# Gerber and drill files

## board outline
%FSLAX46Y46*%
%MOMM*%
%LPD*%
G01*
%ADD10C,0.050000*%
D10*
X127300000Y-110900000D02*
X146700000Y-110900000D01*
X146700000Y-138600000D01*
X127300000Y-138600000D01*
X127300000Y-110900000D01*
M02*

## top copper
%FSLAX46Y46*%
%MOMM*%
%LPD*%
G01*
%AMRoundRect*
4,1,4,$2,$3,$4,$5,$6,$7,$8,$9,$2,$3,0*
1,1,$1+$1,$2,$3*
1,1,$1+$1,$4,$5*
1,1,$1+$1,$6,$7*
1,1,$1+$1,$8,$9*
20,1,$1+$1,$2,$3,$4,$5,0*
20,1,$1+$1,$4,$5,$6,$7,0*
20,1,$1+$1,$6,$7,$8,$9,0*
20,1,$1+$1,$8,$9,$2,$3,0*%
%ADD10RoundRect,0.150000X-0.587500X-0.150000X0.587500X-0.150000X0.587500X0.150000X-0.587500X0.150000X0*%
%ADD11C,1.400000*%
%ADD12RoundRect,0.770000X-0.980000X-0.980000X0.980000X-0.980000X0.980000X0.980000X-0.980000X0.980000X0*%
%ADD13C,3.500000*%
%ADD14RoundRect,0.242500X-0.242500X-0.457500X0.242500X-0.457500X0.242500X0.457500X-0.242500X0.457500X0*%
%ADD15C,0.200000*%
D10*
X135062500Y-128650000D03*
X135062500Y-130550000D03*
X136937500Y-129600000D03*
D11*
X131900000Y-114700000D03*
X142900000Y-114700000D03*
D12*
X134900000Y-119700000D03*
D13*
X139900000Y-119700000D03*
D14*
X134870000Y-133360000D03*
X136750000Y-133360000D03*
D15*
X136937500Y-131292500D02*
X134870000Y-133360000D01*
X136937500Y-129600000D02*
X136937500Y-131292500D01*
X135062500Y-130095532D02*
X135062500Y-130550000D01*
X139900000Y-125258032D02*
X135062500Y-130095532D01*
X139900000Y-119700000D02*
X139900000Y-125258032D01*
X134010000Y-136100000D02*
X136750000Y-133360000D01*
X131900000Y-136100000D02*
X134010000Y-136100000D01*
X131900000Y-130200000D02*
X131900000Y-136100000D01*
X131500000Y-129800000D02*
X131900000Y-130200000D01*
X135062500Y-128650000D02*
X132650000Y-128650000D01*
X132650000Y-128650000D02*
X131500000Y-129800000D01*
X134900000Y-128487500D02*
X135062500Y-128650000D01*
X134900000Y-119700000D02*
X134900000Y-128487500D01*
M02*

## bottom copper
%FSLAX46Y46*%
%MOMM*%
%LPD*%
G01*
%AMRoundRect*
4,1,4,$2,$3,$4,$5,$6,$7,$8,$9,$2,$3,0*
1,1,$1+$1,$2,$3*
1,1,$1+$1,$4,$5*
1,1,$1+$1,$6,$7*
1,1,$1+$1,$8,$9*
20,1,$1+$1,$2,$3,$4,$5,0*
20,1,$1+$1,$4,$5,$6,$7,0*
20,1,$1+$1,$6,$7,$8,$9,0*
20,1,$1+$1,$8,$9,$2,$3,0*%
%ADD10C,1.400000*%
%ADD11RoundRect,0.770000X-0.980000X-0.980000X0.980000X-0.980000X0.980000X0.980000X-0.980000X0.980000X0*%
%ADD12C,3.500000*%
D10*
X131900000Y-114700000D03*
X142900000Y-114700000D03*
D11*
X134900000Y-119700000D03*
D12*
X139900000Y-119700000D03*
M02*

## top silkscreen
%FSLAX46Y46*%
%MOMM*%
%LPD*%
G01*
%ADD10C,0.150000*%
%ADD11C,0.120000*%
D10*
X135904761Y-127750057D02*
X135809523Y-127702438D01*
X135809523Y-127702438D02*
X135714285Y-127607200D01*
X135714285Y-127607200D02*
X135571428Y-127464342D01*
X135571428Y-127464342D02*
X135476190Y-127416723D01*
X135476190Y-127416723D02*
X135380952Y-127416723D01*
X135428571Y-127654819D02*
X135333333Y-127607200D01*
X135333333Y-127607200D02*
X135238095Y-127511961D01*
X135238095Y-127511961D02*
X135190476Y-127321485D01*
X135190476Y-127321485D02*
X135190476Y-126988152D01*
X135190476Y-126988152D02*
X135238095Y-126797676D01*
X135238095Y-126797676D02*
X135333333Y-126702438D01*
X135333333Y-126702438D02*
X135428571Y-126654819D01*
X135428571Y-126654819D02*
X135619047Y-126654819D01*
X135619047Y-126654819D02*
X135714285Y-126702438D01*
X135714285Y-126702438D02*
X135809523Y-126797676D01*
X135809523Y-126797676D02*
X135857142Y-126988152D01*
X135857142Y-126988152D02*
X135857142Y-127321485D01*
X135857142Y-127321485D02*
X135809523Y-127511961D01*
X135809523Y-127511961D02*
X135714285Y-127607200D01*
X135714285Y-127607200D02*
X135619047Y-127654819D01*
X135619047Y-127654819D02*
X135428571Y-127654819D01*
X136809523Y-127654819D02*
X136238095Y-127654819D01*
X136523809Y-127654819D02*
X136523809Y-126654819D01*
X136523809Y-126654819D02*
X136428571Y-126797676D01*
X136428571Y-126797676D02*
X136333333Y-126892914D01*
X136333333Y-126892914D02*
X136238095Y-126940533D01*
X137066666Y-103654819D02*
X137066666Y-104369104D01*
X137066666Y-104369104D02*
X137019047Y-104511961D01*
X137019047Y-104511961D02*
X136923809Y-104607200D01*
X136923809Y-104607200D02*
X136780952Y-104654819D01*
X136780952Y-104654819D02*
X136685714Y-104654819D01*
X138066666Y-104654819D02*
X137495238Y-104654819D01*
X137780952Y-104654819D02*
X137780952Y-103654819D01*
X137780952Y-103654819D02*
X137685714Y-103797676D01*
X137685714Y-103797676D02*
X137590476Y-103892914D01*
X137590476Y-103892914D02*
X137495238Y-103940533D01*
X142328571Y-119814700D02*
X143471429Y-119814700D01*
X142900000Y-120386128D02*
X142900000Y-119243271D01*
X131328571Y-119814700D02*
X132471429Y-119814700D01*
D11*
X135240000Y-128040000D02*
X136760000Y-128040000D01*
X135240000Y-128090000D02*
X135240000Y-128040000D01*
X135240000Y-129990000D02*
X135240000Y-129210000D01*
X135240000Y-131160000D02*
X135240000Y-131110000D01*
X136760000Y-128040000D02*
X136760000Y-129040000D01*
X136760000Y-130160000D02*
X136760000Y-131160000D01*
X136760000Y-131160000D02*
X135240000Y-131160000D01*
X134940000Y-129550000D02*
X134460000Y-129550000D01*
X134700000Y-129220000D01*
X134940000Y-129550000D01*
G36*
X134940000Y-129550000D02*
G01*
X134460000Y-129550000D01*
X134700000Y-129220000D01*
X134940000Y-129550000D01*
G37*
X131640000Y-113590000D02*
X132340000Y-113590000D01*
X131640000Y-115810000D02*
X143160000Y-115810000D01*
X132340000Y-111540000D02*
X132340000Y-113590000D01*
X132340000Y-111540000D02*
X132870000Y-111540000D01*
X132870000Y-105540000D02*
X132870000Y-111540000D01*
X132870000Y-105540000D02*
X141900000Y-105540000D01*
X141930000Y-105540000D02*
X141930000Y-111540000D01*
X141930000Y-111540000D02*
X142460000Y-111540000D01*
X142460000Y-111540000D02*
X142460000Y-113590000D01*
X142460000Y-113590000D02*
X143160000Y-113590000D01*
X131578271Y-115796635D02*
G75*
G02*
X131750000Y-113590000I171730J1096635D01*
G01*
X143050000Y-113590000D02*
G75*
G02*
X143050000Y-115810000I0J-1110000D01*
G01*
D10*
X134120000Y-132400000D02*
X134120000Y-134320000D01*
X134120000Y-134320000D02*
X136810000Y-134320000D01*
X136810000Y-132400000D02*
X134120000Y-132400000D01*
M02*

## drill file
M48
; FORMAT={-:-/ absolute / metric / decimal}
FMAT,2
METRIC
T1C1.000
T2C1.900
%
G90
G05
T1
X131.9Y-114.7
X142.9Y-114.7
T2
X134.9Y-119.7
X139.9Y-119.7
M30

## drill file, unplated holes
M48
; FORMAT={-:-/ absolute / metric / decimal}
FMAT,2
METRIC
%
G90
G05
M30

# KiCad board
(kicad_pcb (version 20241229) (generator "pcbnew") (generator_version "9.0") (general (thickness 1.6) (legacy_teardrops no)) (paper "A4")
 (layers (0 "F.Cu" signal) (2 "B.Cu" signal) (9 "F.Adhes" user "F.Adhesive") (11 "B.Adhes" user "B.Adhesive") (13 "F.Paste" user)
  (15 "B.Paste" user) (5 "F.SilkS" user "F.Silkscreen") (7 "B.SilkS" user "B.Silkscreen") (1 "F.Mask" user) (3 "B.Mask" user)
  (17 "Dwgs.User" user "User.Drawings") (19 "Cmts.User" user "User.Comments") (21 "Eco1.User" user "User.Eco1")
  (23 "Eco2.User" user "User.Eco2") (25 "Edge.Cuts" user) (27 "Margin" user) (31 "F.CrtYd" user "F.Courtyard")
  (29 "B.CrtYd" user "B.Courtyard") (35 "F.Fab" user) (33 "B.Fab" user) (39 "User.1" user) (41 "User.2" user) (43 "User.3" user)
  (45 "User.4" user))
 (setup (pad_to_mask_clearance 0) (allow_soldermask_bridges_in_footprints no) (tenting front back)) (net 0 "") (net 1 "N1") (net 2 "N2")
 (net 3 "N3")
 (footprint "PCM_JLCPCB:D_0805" (layer "F.Cu") (at 135.81 133.36)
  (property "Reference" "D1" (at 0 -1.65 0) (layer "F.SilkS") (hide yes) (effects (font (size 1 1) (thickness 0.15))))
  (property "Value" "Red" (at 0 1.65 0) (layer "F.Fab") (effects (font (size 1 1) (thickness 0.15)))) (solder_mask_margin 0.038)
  (fp_line (start -1.69 -0.96) (end -1.69 0.96) (stroke (width 0.15) (type solid)) (layer "F.SilkS"))
  (fp_line (start -1.69 0.96) (end 1 0.96) (stroke (width 0.15) (type solid)) (layer "F.SilkS"))
  (fp_line (start 1 -0.96) (end -1.69 -0.96) (stroke (width 0.15) (type solid)) (layer "F.SilkS"))
  (pad "1" smd roundrect (at -0.94 0) (size 0.97 1.4) (layers "F.Cu" "F.Mask" "F.Paste") (roundrect_rratio 0.25) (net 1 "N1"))
  (pad "2" smd roundrect (at 0.94 0) (size 0.97 1.4) (layers "F.Cu" "F.Mask" "F.Paste") (roundrect_rratio 0.25) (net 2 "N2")))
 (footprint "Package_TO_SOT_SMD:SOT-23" (layer "F.Cu") (at 136 129.6)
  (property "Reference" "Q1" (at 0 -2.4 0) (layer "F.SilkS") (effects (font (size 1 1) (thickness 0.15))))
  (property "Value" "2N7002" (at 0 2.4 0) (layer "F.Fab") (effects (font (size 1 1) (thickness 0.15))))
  (fp_line (start -0.76 -1.56) (end 0.76 -1.56) (stroke (width 0.12) (type solid)) (layer "F.SilkS"))
  (fp_line (start -0.76 -1.51) (end -0.76 -1.56) (stroke (width 0.12) (type solid)) (layer "F.SilkS"))
  (fp_line (start -0.76 0.39) (end -0.76 -0.39) (stroke (width 0.12) (type solid)) (layer "F.SilkS"))
  (fp_line (start -0.76 1.56) (end -0.76 1.51) (stroke (width 0.12) (type solid)) (layer "F.SilkS"))
  (fp_line (start 0.76 -1.56) (end 0.76 -0.56) (stroke (width 0.12) (type solid)) (layer "F.SilkS"))
  (fp_line (start 0.76 0.56) (end 0.76 1.56) (stroke (width 0.12) (type solid)) (layer "F.SilkS"))
  (fp_line (start 0.76 1.56) (end -0.76 1.56) (stroke (width 0.12) (type solid)) (layer "F.SilkS"))
  (fp_poly (pts (xy -1.3 -0.38) (xy -1.06 -0.05) (xy -1.54 -0.05)) (stroke (width 0.12) (type solid)) (fill yes) (layer "F.SilkS"))
  (pad "1" smd roundrect (at -0.9375 -0.95) (size 1.475 0.6) (layers "F.Cu" "F.Mask" "F.Paste") (roundrect_rratio 0.25) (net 2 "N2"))
  (pad "2" smd roundrect (at -0.9375 0.95) (size 1.475 0.6) (layers "F.Cu" "F.Mask" "F.Paste") (roundrect_rratio 0.25) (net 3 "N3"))
  (pad "3" smd roundrect (at 0.9375 0) (size 1.475 0.6) (layers "F.Cu" "F.Mask" "F.Paste") (roundrect_rratio 0.25) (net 1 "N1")))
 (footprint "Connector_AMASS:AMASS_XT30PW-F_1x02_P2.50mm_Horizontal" (layer "F.Cu") (at 134.9 119.7)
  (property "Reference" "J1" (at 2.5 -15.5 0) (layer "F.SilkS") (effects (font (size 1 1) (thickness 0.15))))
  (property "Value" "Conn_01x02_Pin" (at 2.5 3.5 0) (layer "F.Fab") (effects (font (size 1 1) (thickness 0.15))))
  (fp_line (start -3.26 -6.11) (end -2.56 -6.11) (stroke (width 0.12) (type solid)) (layer "F.SilkS"))
  (fp_line (start -3.26 -3.89) (end 8.26 -3.89) (stroke (width 0.12) (type solid)) (layer "F.SilkS"))
  (fp_line (start -2.56 -8.16) (end -2.56 -6.11) (stroke (width 0.12) (type solid)) (layer "F.SilkS"))
  (fp_line (start -2.56 -8.16) (end -2.03 -8.16) (stroke (width 0.12) (type solid)) (layer "F.SilkS"))
  (fp_line (start -2.03 -14.16) (end -2.03 -8.16) (stroke (width 0.12) (type solid)) (layer "F.SilkS"))
  (fp_line (start -2.03 -14.16) (end 7 -14.16) (stroke (width 0.12) (type solid)) (layer "F.SilkS"))
  (fp_line (start 7.03 -14.16) (end 7.03 -8.16) (stroke (width 0.12) (type solid)) (layer "F.SilkS"))
  (fp_line (start 7.03 -8.16) (end 7.56 -8.16) (stroke (width 0.12) (type solid)) (layer "F.SilkS"))
  (fp_line (start 7.56 -8.16) (end 7.56 -6.11) (stroke (width 0.12) (type solid)) (layer "F.SilkS"))
  (fp_line (start 7.56 -6.11) (end 8.26 -6.11) (stroke (width 0.12) (type solid)) (layer "F.SilkS"))
  (fp_arc (start -3.321729 -3.903365) (mid -4.256653 -5.086124) (end -3.15 -6.11) (stroke (width 0.12) (type solid)) (layer "F.SilkS"))
  (fp_arc (start 8.15 -6.11) (mid 9.26 -5) (end 8.15 -3.89) (stroke (width 0.12) (type solid)) (layer "F.SilkS"))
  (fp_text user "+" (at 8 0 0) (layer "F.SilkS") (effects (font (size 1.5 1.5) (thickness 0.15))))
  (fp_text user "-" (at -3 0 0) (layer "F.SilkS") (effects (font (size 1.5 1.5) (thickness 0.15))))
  (pad "" thru_hole circle (at -3 -5 90) (size 1.4 1.4) (drill 1) (layers "*.Cu" "*.Mask") (remove_unused_layers no))
  (pad "" thru_hole circle (at 8 -5) (size 1.4 1.4) (drill 1) (layers "*.Cu" "*.Mask") (remove_unused_layers no))
  (pad "1" thru_hole roundrect (at 0 0) (size 3.5 3.5) (drill 1.9) (layers "*.Cu" "*.Mask") (remove_unused_layers no)
   (roundrect_rratio 0.22) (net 2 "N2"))
  (pad "2" thru_hole circle (at 5 0) (size 3.5 3.5) (drill 1.9) (layers "*.Cu" "*.Mask") (remove_unused_layers no) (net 3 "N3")))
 (gr_rect (start 127.3 110.9) (end 146.7 138.6) (stroke (width 0.05) (type default)) (fill no) (layer "Edge.Cuts"))
 (segment (start 134.9 119.7) (end 134.9 128.4875) (width 0.2) (layer "F.Cu") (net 2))
 (segment (start 131.9 130.2) (end 131.9 136.1) (width 0.2) (layer "F.Cu") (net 2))
 (segment (start 134.9 128.4875) (end 135.0625 128.65) (width 0.2) (layer "F.Cu") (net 2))
 (segment (start 132.65 128.65) (end 131.5 129.8) (width 0.2) (layer "F.Cu") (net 2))
 (segment (start 134.01 136.1) (end 136.75 133.36) (width 0.2) (layer "F.Cu") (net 2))
 (segment (start 131.9 136.1) (end 134.01 136.1) (width 0.2) (layer "F.Cu") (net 2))
 (segment (start 131.5 129.8) (end 131.9 130.2) (width 0.2) (layer "F.Cu") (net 2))
 (segment (start 135.0625 128.65) (end 132.65 128.65) (width 0.2) (layer "F.Cu") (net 2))
 (segment (start 136.9375 131.2925) (end 134.87 133.36) (width 0.2) (layer "F.Cu") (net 1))
 (segment (start 136.9375 129.6) (end 136.9375 131.2925) (width 0.2) (layer "F.Cu") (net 1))
 (segment (start 139.9 125.258032) (end 135.0625 130.095532) (width 0.2) (layer "F.Cu") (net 3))
 (segment (start 135.0625 130.095532) (end 135.0625 130.55) (width 0.2) (layer "F.Cu") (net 3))
 (segment (start 139.9 119.7) (end 139.9 125.258032) (width 0.2) (layer "F.Cu") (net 3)))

